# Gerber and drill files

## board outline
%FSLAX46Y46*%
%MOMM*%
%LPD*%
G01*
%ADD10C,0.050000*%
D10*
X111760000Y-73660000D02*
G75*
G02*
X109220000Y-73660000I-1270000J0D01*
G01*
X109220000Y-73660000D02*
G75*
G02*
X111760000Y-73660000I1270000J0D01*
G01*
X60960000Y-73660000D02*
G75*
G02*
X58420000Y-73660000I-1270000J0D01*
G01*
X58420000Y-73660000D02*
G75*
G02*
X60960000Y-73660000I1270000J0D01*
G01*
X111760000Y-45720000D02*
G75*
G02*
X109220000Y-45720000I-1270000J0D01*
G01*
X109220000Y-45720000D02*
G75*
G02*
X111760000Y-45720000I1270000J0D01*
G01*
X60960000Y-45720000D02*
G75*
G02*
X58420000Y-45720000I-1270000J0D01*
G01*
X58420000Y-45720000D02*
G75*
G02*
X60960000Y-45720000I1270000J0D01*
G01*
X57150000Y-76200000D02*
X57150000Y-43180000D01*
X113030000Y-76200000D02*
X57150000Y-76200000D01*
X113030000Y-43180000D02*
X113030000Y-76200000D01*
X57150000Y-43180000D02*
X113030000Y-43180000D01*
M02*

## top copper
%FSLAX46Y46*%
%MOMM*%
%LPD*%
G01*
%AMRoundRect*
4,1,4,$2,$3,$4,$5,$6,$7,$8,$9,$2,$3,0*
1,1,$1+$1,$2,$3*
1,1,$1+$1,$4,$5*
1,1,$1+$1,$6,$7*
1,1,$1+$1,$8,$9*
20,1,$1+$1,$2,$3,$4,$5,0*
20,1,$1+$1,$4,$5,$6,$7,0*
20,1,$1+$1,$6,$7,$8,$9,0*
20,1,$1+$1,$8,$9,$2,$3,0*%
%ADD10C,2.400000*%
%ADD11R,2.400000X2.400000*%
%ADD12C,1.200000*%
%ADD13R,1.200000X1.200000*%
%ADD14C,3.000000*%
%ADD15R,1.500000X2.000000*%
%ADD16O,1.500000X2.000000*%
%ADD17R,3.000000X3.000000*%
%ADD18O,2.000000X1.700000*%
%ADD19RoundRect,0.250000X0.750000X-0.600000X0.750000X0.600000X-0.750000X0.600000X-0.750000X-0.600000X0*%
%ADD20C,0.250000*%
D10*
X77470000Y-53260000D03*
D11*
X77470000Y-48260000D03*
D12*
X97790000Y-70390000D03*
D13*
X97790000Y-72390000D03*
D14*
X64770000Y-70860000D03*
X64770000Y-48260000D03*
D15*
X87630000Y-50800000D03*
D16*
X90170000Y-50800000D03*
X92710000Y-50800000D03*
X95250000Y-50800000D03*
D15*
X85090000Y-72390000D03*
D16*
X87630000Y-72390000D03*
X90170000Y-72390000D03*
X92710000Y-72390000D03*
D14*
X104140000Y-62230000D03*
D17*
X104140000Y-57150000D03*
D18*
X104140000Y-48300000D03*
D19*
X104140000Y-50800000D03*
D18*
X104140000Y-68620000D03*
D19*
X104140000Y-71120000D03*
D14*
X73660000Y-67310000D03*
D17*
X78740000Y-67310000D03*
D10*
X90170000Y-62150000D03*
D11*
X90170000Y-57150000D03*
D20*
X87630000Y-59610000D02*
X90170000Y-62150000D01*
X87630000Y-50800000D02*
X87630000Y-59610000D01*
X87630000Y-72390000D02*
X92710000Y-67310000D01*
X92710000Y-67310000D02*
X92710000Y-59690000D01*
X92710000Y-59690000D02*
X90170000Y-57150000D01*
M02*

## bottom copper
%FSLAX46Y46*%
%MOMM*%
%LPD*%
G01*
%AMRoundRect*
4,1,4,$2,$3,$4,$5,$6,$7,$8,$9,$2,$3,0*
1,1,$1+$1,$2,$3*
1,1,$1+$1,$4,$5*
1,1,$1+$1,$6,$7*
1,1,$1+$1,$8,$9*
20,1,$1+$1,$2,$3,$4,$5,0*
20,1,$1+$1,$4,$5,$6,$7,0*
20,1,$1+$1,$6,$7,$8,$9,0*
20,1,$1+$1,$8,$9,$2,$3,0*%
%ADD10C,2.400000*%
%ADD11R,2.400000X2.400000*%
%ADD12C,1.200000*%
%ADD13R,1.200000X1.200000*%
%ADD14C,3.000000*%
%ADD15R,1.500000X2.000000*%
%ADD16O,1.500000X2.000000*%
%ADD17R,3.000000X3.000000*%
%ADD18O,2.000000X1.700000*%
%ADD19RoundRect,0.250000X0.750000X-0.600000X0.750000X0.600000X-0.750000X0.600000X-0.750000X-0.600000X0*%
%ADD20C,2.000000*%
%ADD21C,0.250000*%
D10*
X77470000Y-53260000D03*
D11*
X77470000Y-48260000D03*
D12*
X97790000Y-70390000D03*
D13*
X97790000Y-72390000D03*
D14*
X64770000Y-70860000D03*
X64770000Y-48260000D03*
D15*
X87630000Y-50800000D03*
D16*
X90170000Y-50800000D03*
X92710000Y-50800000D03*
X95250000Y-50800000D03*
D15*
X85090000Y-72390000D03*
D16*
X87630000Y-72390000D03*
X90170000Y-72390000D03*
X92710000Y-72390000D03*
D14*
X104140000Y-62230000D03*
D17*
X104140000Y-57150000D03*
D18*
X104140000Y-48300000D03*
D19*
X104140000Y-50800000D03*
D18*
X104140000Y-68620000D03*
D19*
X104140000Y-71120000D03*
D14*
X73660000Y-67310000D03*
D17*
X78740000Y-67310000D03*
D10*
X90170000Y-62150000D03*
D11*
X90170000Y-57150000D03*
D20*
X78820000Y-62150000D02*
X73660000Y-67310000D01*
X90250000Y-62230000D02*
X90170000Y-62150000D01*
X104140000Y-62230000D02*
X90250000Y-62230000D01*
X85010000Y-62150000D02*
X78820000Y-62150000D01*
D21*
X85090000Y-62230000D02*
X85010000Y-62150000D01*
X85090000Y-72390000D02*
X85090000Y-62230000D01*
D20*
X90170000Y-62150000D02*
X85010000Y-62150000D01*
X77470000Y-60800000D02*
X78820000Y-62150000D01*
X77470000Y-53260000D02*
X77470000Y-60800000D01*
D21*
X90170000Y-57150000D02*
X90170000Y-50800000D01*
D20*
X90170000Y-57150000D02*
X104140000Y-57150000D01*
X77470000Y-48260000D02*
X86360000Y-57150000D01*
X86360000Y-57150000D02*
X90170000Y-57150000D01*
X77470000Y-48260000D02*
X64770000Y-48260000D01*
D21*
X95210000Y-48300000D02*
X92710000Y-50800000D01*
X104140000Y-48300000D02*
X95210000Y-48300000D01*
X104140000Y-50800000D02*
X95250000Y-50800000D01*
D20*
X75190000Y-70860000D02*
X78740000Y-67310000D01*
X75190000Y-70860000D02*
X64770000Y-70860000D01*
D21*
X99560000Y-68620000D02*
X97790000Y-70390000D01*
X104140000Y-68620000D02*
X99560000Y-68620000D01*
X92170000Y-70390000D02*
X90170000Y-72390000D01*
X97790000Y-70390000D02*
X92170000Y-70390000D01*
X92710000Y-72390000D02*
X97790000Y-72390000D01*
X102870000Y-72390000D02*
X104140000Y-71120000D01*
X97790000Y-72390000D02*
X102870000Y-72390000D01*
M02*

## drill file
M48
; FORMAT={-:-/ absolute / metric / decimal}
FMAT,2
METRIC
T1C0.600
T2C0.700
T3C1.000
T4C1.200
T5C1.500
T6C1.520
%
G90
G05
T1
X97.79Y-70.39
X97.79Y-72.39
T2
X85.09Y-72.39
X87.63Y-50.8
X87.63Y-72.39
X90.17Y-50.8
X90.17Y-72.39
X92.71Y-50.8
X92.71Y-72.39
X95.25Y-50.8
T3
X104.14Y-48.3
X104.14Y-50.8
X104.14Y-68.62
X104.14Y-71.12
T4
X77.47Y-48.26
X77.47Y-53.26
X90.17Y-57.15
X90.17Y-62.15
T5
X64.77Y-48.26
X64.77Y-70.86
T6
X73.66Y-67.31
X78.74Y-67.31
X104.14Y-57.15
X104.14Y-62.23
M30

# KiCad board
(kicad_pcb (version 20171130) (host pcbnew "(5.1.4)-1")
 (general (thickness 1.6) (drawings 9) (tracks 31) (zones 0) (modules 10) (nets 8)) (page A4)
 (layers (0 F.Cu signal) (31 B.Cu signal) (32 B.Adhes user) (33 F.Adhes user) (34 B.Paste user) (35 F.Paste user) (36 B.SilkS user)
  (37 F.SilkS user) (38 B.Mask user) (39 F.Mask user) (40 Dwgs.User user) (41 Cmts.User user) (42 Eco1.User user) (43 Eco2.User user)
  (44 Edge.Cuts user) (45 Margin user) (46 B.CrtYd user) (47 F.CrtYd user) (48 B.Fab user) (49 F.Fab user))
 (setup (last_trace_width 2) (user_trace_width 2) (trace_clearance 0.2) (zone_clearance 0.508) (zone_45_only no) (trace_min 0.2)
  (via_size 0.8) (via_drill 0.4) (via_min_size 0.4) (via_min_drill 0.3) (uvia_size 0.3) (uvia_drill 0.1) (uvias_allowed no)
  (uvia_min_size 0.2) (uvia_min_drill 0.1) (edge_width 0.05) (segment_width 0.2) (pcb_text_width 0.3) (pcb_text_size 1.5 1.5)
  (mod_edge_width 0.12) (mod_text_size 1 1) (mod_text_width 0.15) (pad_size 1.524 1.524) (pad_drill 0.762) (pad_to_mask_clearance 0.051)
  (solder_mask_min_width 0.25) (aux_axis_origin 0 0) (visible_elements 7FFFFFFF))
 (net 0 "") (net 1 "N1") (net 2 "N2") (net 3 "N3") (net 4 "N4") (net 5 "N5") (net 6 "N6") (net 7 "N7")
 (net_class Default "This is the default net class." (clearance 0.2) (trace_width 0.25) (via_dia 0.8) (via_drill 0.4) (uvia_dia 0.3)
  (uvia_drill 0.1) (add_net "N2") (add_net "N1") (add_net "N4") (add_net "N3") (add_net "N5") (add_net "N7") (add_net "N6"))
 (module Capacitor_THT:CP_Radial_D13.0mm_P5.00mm (layer F.Cu) (at 77.47 48.26 270)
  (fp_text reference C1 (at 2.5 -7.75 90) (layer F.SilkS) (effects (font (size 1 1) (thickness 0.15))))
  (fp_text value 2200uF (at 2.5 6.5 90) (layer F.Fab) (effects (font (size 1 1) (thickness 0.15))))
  (pad 2 thru_hole circle (at 5 0 270) (size 2.4 2.4) (drill 1.2) (layers *.Cu *.Mask) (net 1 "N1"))
  (pad 1 thru_hole rect (at 0 0 270) (size 2.4 2.4) (drill 1.2) (layers *.Cu *.Mask) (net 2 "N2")))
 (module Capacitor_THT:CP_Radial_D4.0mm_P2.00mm (layer F.Cu) (at 97.79 72.39 90)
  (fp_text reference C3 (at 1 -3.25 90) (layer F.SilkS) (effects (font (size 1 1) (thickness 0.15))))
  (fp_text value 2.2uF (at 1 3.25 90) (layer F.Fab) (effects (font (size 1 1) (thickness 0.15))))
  (pad 2 thru_hole circle (at 2 0 90) (size 1.2 1.2) (drill 0.6) (layers *.Cu *.Mask) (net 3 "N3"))
  (pad 1 thru_hole rect (at 0 0 90) (size 1.2 1.2) (drill 0.6) (layers *.Cu *.Mask) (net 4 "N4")))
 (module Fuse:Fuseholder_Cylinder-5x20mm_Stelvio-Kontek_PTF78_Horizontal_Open (layer F.Cu) (at 64.77 48.26 270)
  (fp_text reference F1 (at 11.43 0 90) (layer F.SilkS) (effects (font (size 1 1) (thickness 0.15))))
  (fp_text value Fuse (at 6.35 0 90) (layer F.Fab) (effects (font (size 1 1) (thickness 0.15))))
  (pad 2 thru_hole circle (at 22.6 0 270) (size 3 3) (drill 1.5) (layers *.Cu *.Mask) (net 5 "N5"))
  (pad 1 thru_hole circle (at 0 0 270) (size 3 3) (drill 1.5) (layers *.Cu *.Mask) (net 2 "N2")))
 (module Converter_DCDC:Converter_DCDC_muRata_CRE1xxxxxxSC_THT (layer F.Cu) (at 87.63 50.8 90)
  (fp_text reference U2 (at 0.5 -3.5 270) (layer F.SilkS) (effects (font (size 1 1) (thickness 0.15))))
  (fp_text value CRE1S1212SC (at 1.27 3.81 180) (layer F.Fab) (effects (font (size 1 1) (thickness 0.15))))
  (pad 1 thru_hole rect (at 0 0) (size 1.5 2) (drill 0.7) (layers *.Cu *.Mask) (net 1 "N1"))
  (pad 2 thru_hole oval (at 0 2.54) (size 1.5 2) (drill 0.7) (layers *.Cu *.Mask) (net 2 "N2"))
  (pad 3 thru_hole oval (at 0 5.08) (size 1.5 2) (drill 0.7) (layers *.Cu *.Mask) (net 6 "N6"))
  (pad 4 thru_hole oval (at 0 7.62) (size 1.5 2) (drill 0.7) (layers *.Cu *.Mask) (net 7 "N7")))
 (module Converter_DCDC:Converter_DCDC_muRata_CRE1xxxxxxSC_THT (layer F.Cu) (at 85.09 72.39 90)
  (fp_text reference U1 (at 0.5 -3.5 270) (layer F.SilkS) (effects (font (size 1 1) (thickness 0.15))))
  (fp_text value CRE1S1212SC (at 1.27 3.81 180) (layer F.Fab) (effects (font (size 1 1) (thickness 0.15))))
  (pad 1 thru_hole rect (at 0 0) (size 1.5 2) (drill 0.7) (layers *.Cu *.Mask) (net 1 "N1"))
  (pad 2 thru_hole oval (at 0 2.54) (size 1.5 2) (drill 0.7) (layers *.Cu *.Mask) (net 2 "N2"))
  (pad 3 thru_hole oval (at 0 5.08) (size 1.5 2) (drill 0.7) (layers *.Cu *.Mask) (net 3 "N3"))
  (pad 4 thru_hole oval (at 0 7.62) (size 1.5 2) (drill 0.7) (layers *.Cu *.Mask) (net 4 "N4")))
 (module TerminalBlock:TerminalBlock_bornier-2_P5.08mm (layer F.Cu) (at 104.14 57.15 270)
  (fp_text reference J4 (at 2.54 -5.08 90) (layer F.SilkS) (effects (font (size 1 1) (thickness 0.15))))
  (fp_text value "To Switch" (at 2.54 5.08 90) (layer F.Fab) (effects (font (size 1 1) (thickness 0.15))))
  (pad 2 thru_hole circle (at 5.08 0 270) (size 3 3) (drill 1.52) (layers *.Cu *.Mask) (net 1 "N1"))
  (pad 1 thru_hole rect (at 0 0 270) (size 3 3) (drill 1.52) (layers *.Cu *.Mask) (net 2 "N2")))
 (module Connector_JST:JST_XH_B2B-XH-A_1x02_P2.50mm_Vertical (layer F.Cu) (at 104.14 50.8 90)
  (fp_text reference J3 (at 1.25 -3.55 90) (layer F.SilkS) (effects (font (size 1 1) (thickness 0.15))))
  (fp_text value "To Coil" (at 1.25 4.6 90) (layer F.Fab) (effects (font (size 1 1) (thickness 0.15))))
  (pad 2 thru_hole oval (at 2.5 0 90) (size 1.7 2) (drill 1) (layers *.Cu *.Mask) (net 6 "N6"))
  (pad 1 thru_hole roundrect (at 0 0 90) (size 1.7 2) (drill 1) (layers *.Cu *.Mask) (roundrect_rratio 0.147059) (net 7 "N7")))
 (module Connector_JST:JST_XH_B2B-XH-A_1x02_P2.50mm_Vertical (layer F.Cu) (at 104.14 71.12 90)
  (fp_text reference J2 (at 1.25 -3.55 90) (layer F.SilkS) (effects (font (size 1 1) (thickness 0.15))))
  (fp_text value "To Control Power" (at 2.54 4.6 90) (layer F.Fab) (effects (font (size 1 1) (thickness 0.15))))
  (pad 2 thru_hole oval (at 2.5 0 90) (size 1.7 2) (drill 1) (layers *.Cu *.Mask) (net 3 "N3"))
  (pad 1 thru_hole roundrect (at 0 0 90) (size 1.7 2) (drill 1) (layers *.Cu *.Mask) (roundrect_rratio 0.147059) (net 4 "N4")))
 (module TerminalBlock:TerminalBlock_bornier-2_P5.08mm (layer F.Cu) (at 78.74 67.31 180)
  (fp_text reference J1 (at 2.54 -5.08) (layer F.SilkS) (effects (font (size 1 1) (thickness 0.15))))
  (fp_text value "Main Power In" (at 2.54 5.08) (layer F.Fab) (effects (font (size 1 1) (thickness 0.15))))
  (pad 2 thru_hole circle (at 5.08 0 180) (size 3 3) (drill 1.52) (layers *.Cu *.Mask) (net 1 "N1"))
  (pad 1 thru_hole rect (at 0 0 180) (size 3 3) (drill 1.52) (layers *.Cu *.Mask) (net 5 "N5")))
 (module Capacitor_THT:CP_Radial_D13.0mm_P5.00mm (layer F.Cu) (at 90.17 57.15 270)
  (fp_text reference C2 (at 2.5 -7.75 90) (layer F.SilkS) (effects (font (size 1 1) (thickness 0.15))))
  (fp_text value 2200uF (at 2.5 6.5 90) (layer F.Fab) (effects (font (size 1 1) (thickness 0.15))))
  (pad 2 thru_hole circle (at 5 0 270) (size 2.4 2.4) (drill 1.2) (layers *.Cu *.Mask) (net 1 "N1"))
  (pad 1 thru_hole rect (at 0 0 270) (size 2.4 2.4) (drill 1.2) (layers *.Cu *.Mask) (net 2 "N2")))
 (gr_circle (center 110.49 73.66) (end 111.76 73.66) (layer Edge.Cuts) (width 0.05))
 (gr_circle (center 59.69 73.66) (end 58.42 73.66) (layer Edge.Cuts) (width 0.05))
 (gr_circle (center 110.49 45.72) (end 111.76 45.72) (layer Edge.Cuts) (width 0.05))
 (gr_circle (center 59.69 45.72) (end 60.96 45.72) (layer Edge.Cuts) (width 0.05))
 (gr_line (start 57.15 76.2) (end 57.15 43.18) (layer Edge.Cuts) (width 0.05))
 (gr_line (start 113.03 76.2) (end 57.15 76.2) (layer Edge.Cuts) (width 0.05))
 (gr_line (start 113.03 43.18) (end 113.03 76.2) (layer Edge.Cuts) (width 0.05))
 (gr_line (start 57.15 43.18) (end 113.03 43.18) (layer Edge.Cuts) (width 0.05))
 (segment (start 78.82 62.15) (end 73.66 67.31) (width 2) (layer B.Cu) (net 1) (status 20))
 (segment (start 90.25 62.23) (end 90.17 62.15) (width 2) (layer B.Cu) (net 1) (status 30))
 (segment (start 104.14 62.23) (end 90.25 62.23) (width 2) (layer B.Cu) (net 1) (status 30))
 (segment (start 85.01 62.15) (end 78.82 62.15) (width 2) (layer B.Cu) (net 1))
 (segment (start 85.09 62.23) (end 85.01 62.15) (width 0.25) (layer B.Cu) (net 1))
 (segment (start 85.09 72.39) (end 85.09 62.23) (width 0.25) (layer B.Cu) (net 1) (status 10))
 (segment (start 90.17 62.15) (end 85.01 62.15) (width 2) (layer B.Cu) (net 1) (status 10))
 (segment (start 87.63 59.61) (end 90.17 62.15) (width 0.25) (layer F.Cu) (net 1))
 (segment (start 87.63 50.8) (end 87.63 59.61) (width 0.25) (layer F.Cu) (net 1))
 (segment (start 77.47 60.8) (end 78.82 62.15) (width 2) (layer B.Cu) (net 1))
 (segment (start 77.47 53.26) (end 77.47 60.8) (width 2) (layer B.Cu) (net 1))
 (segment (start 90.17 57.15) (end 90.17 50.8) (width 0.25) (layer B.Cu) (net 2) (status 30))
 (segment (start 90.17 57.15) (end 104.14 57.15) (width 2) (layer B.Cu) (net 2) (status 30))
 (segment (start 87.63 72.39) (end 92.71 67.31) (width 0.25) (layer F.Cu) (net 2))
 (segment (start 92.71 67.31) (end 92.71 59.69) (width 0.25) (layer F.Cu) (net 2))
 (segment (start 92.71 59.69) (end 90.17 57.15) (width 0.25) (layer F.Cu) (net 2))
 (segment (start 77.47 48.26) (end 86.36 57.15) (width 2) (layer B.Cu) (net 2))
 (segment (start 86.36 57.15) (end 90.17 57.15) (width 2) (layer B.Cu) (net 2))
 (segment (start 77.47 48.26) (end 64.77 48.26) (width 2) (layer B.Cu) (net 2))
 (segment (start 95.21 48.3) (end 92.71 50.8) (width 0.25) (layer B.Cu) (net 6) (status 20))
 (segment (start 104.14 48.3) (end 95.21 48.3) (width 0.25) (layer B.Cu) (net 6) (status 10))
 (segment (start 104.14 50.8) (end 95.25 50.8) (width 0.25) (layer B.Cu) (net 7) (status 30))
 (segment (start 75.19 70.86) (end 78.74 67.31) (width 2) (layer B.Cu) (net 5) (status 20))
 (segment (start 75.19 70.86) (end 64.77 70.86) (width 2) (layer B.Cu) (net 5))
 (segment (start 99.56 68.62) (end 97.79 70.39) (width 0.25) (layer B.Cu) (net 3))
 (segment (start 104.14 68.62) (end 99.56 68.62) (width 0.25) (layer B.Cu) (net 3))
 (segment (start 92.17 70.39) (end 90.17 72.39) (width 0.25) (layer B.Cu) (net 3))
 (segment (start 97.79 70.39) (end 92.17 70.39) (width 0.25) (layer B.Cu) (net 3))
 (segment (start 92.71 72.39) (end 97.79 72.39) (width 0.25) (layer B.Cu) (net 4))
 (segment (start 102.87 72.39) (end 104.14 71.12) (width 0.25) (layer B.Cu) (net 4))
 (segment (start 97.79 72.39) (end 102.87 72.39) (width 0.25) (layer B.Cu) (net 4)))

